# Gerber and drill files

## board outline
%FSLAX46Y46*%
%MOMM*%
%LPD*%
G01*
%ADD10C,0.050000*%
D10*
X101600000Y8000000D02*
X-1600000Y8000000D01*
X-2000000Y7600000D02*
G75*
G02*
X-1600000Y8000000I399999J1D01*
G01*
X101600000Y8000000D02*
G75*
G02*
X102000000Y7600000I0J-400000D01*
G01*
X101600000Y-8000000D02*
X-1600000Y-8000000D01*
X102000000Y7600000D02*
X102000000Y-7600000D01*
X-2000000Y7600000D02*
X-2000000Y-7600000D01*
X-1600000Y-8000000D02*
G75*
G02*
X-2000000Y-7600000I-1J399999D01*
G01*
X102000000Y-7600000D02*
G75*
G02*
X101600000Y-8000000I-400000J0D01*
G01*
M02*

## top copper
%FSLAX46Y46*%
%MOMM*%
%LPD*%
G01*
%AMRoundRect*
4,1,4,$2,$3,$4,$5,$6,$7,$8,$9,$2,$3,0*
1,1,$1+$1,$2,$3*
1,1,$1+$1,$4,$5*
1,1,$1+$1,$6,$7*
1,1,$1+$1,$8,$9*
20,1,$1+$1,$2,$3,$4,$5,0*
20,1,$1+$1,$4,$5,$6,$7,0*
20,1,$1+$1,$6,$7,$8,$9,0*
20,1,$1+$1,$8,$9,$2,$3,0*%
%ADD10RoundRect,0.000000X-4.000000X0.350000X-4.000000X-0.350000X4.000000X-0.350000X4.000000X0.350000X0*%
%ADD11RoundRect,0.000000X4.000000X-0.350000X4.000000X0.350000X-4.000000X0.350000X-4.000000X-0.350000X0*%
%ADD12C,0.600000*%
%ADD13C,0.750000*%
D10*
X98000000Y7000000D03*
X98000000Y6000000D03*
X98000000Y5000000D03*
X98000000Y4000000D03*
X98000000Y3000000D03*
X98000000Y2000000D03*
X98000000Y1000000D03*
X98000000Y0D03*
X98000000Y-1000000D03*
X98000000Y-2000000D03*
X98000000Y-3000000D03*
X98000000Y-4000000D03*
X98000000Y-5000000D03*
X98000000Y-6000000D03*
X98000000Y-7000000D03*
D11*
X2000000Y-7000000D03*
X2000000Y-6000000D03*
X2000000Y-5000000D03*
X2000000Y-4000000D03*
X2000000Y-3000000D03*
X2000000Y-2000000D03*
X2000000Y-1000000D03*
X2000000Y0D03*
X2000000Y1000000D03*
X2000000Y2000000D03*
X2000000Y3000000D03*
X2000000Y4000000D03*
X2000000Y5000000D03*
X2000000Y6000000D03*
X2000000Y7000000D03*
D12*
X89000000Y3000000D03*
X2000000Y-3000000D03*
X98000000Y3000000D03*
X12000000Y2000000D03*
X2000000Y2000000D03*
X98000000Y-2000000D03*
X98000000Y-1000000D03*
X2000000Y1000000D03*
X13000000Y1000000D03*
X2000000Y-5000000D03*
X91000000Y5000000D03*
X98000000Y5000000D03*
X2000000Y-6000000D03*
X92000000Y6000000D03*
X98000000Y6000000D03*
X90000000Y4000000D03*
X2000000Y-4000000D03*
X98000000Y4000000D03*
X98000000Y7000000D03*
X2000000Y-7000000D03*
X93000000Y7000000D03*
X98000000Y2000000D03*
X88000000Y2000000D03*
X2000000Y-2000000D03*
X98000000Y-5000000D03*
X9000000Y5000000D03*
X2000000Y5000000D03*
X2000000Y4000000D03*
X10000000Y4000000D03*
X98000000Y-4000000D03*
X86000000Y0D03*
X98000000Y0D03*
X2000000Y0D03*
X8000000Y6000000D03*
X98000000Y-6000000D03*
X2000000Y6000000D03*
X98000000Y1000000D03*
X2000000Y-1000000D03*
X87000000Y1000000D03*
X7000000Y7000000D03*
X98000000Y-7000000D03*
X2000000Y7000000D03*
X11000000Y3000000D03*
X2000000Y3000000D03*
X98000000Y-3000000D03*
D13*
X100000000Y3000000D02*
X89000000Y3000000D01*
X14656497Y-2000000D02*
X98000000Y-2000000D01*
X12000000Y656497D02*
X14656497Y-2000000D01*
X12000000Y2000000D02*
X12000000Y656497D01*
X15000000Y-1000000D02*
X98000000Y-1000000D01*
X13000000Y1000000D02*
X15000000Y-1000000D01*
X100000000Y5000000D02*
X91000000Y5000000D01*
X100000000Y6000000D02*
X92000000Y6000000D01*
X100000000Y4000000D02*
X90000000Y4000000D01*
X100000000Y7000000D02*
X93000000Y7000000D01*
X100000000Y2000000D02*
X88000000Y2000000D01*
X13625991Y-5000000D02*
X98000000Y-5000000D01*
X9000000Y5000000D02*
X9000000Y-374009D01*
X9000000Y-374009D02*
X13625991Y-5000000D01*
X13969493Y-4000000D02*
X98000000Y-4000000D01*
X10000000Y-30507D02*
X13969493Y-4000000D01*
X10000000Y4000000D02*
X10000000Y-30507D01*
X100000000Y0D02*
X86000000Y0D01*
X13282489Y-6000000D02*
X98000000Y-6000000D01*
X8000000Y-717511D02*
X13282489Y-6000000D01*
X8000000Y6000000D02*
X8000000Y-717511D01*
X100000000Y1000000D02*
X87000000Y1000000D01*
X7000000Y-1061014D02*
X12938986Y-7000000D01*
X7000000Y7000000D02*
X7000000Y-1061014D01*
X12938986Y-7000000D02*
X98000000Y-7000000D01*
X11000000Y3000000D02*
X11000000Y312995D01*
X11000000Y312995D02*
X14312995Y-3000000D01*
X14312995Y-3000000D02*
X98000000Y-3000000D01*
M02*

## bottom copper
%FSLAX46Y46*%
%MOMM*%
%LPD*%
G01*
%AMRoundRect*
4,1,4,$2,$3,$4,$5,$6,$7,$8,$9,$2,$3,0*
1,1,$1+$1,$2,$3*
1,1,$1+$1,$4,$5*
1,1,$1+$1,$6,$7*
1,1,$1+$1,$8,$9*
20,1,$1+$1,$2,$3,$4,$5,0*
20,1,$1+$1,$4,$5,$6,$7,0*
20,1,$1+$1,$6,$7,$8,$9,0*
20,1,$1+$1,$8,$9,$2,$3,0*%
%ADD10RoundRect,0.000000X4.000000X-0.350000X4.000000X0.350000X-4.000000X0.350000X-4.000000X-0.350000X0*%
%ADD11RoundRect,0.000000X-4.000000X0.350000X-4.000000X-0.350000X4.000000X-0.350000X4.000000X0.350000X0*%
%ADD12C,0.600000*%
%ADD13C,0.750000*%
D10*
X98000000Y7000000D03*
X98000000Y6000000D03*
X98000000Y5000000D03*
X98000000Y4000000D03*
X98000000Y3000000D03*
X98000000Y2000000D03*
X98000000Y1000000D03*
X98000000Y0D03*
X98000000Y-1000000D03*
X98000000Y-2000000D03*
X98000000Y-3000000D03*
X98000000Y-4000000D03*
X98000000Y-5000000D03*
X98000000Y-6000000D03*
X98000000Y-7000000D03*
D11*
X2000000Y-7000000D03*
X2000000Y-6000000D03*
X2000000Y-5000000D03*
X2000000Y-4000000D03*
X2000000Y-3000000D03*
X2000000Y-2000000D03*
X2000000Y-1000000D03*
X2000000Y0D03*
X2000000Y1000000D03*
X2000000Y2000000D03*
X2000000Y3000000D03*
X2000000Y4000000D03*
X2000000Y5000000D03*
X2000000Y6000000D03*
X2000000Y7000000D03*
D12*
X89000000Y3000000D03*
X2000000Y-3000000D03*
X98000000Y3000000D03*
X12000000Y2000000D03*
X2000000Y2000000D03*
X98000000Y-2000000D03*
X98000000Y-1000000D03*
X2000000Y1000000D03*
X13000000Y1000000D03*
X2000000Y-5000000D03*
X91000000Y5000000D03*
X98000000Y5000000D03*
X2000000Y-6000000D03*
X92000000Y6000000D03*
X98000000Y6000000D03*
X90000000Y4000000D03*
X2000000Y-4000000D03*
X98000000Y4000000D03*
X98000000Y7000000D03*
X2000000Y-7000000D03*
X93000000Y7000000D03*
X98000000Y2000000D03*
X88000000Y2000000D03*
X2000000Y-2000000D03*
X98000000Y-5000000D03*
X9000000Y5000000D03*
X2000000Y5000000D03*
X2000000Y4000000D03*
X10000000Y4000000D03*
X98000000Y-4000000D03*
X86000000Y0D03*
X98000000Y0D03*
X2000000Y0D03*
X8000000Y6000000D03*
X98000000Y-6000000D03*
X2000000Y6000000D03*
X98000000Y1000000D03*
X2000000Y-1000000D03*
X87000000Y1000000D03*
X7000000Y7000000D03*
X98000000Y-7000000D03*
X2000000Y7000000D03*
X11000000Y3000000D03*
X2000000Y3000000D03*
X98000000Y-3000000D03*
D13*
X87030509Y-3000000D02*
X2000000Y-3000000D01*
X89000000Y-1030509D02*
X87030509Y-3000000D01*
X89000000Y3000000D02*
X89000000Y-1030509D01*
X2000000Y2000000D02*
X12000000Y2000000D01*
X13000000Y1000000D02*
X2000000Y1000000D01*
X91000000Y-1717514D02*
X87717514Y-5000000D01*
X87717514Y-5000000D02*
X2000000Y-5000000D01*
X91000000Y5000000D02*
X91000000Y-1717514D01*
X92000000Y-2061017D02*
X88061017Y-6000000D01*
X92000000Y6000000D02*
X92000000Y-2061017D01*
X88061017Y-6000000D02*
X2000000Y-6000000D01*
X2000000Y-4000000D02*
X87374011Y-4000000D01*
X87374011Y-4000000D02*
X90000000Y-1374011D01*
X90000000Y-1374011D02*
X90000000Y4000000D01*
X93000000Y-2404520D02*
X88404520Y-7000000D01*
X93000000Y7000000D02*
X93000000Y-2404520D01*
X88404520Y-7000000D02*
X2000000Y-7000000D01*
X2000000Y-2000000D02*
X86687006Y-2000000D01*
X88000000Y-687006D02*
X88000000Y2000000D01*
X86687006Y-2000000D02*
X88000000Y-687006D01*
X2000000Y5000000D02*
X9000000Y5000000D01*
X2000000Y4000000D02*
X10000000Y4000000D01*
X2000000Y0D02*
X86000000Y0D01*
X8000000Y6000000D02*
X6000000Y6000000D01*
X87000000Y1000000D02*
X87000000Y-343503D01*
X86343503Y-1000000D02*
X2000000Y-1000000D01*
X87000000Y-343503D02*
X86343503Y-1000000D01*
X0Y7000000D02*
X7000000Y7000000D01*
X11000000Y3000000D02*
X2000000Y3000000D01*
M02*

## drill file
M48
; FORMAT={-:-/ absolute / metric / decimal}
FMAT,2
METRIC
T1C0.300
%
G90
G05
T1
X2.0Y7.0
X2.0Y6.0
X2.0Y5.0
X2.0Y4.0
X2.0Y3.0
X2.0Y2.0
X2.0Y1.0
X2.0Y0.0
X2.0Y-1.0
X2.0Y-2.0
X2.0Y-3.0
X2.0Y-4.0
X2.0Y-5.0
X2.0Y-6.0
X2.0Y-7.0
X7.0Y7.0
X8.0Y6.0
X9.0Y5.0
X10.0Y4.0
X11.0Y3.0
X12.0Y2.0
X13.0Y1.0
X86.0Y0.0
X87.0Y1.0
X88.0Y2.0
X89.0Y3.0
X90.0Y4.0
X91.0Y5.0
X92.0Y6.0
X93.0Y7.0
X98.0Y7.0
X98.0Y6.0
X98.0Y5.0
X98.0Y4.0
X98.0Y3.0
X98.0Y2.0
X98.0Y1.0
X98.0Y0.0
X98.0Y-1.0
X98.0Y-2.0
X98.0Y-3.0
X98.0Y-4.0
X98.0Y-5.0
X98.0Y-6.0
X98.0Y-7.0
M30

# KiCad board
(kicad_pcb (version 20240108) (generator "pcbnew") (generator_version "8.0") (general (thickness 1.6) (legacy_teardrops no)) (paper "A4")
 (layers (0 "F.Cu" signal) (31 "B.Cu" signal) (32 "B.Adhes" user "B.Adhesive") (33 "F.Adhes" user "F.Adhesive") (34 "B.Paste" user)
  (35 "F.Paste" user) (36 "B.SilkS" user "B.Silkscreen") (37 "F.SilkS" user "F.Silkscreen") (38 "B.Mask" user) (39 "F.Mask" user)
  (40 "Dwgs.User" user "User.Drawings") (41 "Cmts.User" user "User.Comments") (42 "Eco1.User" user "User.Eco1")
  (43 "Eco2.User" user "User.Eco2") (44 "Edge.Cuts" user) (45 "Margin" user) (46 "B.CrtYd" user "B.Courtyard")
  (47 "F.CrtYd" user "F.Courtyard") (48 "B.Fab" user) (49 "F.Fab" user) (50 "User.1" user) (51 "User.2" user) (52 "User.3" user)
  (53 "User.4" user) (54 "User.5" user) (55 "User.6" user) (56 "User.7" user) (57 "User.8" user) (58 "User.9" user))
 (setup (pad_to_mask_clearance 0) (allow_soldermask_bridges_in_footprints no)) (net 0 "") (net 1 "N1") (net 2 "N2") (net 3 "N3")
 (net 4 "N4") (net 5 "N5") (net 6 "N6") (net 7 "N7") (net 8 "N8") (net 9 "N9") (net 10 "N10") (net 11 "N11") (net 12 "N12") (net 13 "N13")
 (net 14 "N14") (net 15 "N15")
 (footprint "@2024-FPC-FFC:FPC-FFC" (layer "F.Cu") (at 98 0 -90)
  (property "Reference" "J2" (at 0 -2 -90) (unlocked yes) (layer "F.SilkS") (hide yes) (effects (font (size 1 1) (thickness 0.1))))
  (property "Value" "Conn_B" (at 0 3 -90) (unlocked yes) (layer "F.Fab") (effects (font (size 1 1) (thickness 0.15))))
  (pad "1" smd roundrect (at -7 0 270) (size 0.7 8) (layers "F.Cu" "F.Paste" "B.SilkS" "F.Mask") (roundrect_rratio 0) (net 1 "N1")
   (thermal_bridge_angle 45))
  (pad "1" smd roundrect (at -7 0 90) (size 0.7 8) (layers "B.Cu" "B.Paste" "F.SilkS" "B.Mask") (roundrect_rratio 0) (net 1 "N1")
   (thermal_bridge_angle 45))
  (pad "2" smd roundrect (at -6 0 270) (size 0.7 8) (layers "F.Cu" "F.Paste" "B.SilkS" "F.Mask") (roundrect_rratio 0) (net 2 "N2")
   (thermal_bridge_angle 45))
  (pad "2" smd roundrect (at -6 0 90) (size 0.7 8) (layers "B.Cu" "B.Paste" "F.SilkS" "B.Mask") (roundrect_rratio 0) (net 2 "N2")
   (thermal_bridge_angle 45))
  (pad "3" smd roundrect (at -5 0 270) (size 0.7 8) (layers "F.Cu" "F.Paste" "B.SilkS" "F.Mask") (roundrect_rratio 0) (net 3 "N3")
   (thermal_bridge_angle 45))
  (pad "3" smd roundrect (at -5 0 90) (size 0.7 8) (layers "B.Cu" "B.Paste" "F.SilkS" "B.Mask") (roundrect_rratio 0) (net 3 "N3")
   (thermal_bridge_angle 45))
  (pad "4" smd roundrect (at -4 0 270) (size 0.7 8) (layers "F.Cu" "F.Paste" "B.SilkS" "F.Mask") (roundrect_rratio 0) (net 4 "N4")
   (thermal_bridge_angle 45))
  (pad "4" smd roundrect (at -4 0 90) (size 0.7 8) (layers "B.Cu" "B.Paste" "F.SilkS" "B.Mask") (roundrect_rratio 0) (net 4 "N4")
   (thermal_bridge_angle 45))
  (pad "5" smd roundrect (at -3 0 270) (size 0.7 8) (layers "F.Cu" "F.Paste" "B.SilkS" "F.Mask") (roundrect_rratio 0) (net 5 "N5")
   (thermal_bridge_angle 45))
  (pad "5" smd roundrect (at -3 0 90) (size 0.7 8) (layers "B.Cu" "B.Paste" "F.SilkS" "B.Mask") (roundrect_rratio 0) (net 5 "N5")
   (thermal_bridge_angle 45))
  (pad "6" smd roundrect (at -2 0 270) (size 0.7 8) (layers "F.Cu" "F.Paste" "B.SilkS" "F.Mask") (roundrect_rratio 0) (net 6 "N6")
   (thermal_bridge_angle 45))
  (pad "6" smd roundrect (at -2 0 90) (size 0.7 8) (layers "B.Cu" "B.Paste" "F.SilkS" "B.Mask") (roundrect_rratio 0) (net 6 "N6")
   (thermal_bridge_angle 45))
  (pad "7" smd roundrect (at -1 0 270) (size 0.7 8) (layers "F.Cu" "F.Paste" "B.SilkS" "F.Mask") (roundrect_rratio 0) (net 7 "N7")
   (thermal_bridge_angle 45))
  (pad "7" smd roundrect (at -1 0 90) (size 0.7 8) (layers "B.Cu" "B.Paste" "F.SilkS" "B.Mask") (roundrect_rratio 0) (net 7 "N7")
   (thermal_bridge_angle 45))
  (pad "8" smd roundrect (at 0 0 270) (size 0.7 8) (layers "F.Cu" "F.Paste" "B.SilkS" "F.Mask") (roundrect_rratio 0) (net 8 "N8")
   (thermal_bridge_angle 45))
  (pad "8" smd roundrect (at 0 0 90) (size 0.7 8) (layers "B.Cu" "B.Paste" "F.SilkS" "B.Mask") (roundrect_rratio 0) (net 8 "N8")
   (thermal_bridge_angle 45))
  (pad "9" smd roundrect (at 1 0 270) (size 0.7 8) (layers "F.Cu" "F.Paste" "B.SilkS" "F.Mask") (roundrect_rratio 0) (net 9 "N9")
   (thermal_bridge_angle 45))
  (pad "9" smd roundrect (at 1 0 90) (size 0.7 8) (layers "B.Cu" "B.Paste" "F.SilkS" "B.Mask") (roundrect_rratio 0) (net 9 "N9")
   (thermal_bridge_angle 45))
  (pad "10" smd roundrect (at 2 0 270) (size 0.7 8) (layers "F.Cu" "F.Paste" "B.SilkS" "F.Mask") (roundrect_rratio 0) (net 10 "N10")
   (thermal_bridge_angle 45))
  (pad "10" smd roundrect (at 2 0 90) (size 0.7 8) (layers "B.Cu" "B.Paste" "F.SilkS" "B.Mask") (roundrect_rratio 0) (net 10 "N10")
   (thermal_bridge_angle 45))
  (pad "11" smd roundrect (at 3 0 270) (size 0.7 8) (layers "F.Cu" "F.Paste" "B.SilkS" "F.Mask") (roundrect_rratio 0) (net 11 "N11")
   (thermal_bridge_angle 45))
  (pad "11" smd roundrect (at 3 0 90) (size 0.7 8) (layers "B.Cu" "B.Paste" "F.SilkS" "B.Mask") (roundrect_rratio 0) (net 11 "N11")
   (thermal_bridge_angle 45))
  (pad "12" smd roundrect (at 4 0 270) (size 0.7 8) (layers "F.Cu" "F.Paste" "B.SilkS" "F.Mask") (roundrect_rratio 0) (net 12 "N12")
   (thermal_bridge_angle 45))
  (pad "12" smd roundrect (at 4 0 90) (size 0.7 8) (layers "B.Cu" "B.Paste" "F.SilkS" "B.Mask") (roundrect_rratio 0) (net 12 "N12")
   (thermal_bridge_angle 45))
  (pad "13" smd roundrect (at 5 0 270) (size 0.7 8) (layers "F.Cu" "F.Paste" "B.SilkS" "F.Mask") (roundrect_rratio 0) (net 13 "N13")
   (thermal_bridge_angle 45))
  (pad "13" smd roundrect (at 5 0 90) (size 0.7 8) (layers "B.Cu" "B.Paste" "F.SilkS" "B.Mask") (roundrect_rratio 0) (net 13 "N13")
   (thermal_bridge_angle 45))
  (pad "14" smd roundrect (at 6 0 270) (size 0.7 8) (layers "F.Cu" "F.Paste" "B.SilkS" "F.Mask") (roundrect_rratio 0) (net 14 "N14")
   (thermal_bridge_angle 45))
  (pad "14" smd roundrect (at 6 0 90) (size 0.7 8) (layers "B.Cu" "B.Paste" "F.SilkS" "B.Mask") (roundrect_rratio 0) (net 14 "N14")
   (thermal_bridge_angle 45))
  (pad "15" smd roundrect (at 7 0 270) (size 0.7 8) (layers "F.Cu" "F.Paste" "B.SilkS" "F.Mask") (roundrect_rratio 0) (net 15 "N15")
   (thermal_bridge_angle 45))
  (pad "15" smd roundrect (at 7 0 90) (size 0.7 8) (layers "B.Cu" "B.Paste" "F.SilkS" "B.Mask") (roundrect_rratio 0) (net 15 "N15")
   (thermal_bridge_angle 45)))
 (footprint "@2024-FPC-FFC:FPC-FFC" (layer "F.Cu") (at 2 0 90)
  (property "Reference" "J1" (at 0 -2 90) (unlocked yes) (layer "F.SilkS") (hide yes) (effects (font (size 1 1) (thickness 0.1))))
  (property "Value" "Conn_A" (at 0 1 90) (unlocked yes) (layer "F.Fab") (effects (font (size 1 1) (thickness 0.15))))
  (pad "1" smd roundrect (at -7 0 90) (size 0.7 8) (layers "F.Cu" "F.Paste" "B.SilkS" "F.Mask") (roundrect_rratio 0) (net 1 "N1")
   (thermal_bridge_angle 45))
  (pad "1" smd roundrect (at -7 0 270) (size 0.7 8) (layers "B.Cu" "B.Paste" "F.SilkS" "B.Mask") (roundrect_rratio 0) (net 1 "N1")
   (thermal_bridge_angle 45))
  (pad "2" smd roundrect (at -6 0 90) (size 0.7 8) (layers "F.Cu" "F.Paste" "B.SilkS" "F.Mask") (roundrect_rratio 0) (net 2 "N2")
   (thermal_bridge_angle 45))
  (pad "2" smd roundrect (at -6 0 270) (size 0.7 8) (layers "B.Cu" "B.Paste" "F.SilkS" "B.Mask") (roundrect_rratio 0) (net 2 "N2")
   (thermal_bridge_angle 45))
  (pad "3" smd roundrect (at -5 0 90) (size 0.7 8) (layers "F.Cu" "F.Paste" "B.SilkS" "F.Mask") (roundrect_rratio 0) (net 3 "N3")
   (thermal_bridge_angle 45))
  (pad "3" smd roundrect (at -5 0 270) (size 0.7 8) (layers "B.Cu" "B.Paste" "F.SilkS" "B.Mask") (roundrect_rratio 0) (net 3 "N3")
   (thermal_bridge_angle 45))
  (pad "4" smd roundrect (at -4 0 90) (size 0.7 8) (layers "F.Cu" "F.Paste" "B.SilkS" "F.Mask") (roundrect_rratio 0) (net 4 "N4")
   (thermal_bridge_angle 45))
  (pad "4" smd roundrect (at -4 0 270) (size 0.7 8) (layers "B.Cu" "B.Paste" "F.SilkS" "B.Mask") (roundrect_rratio 0) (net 4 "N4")
   (thermal_bridge_angle 45))
  (pad "5" smd roundrect (at -3 0 90) (size 0.7 8) (layers "F.Cu" "F.Paste" "B.SilkS" "F.Mask") (roundrect_rratio 0) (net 5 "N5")
   (thermal_bridge_angle 45))
  (pad "5" smd roundrect (at -3 0 270) (size 0.7 8) (layers "B.Cu" "B.Paste" "F.SilkS" "B.Mask") (roundrect_rratio 0) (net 5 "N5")
   (thermal_bridge_angle 45))
  (pad "6" smd roundrect (at -2 0 90) (size 0.7 8) (layers "F.Cu" "F.Paste" "B.SilkS" "F.Mask") (roundrect_rratio 0) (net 6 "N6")
   (thermal_bridge_angle 45))
  (pad "6" smd roundrect (at -2 0 270) (size 0.7 8) (layers "B.Cu" "B.Paste" "F.SilkS" "B.Mask") (roundrect_rratio 0) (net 6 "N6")
   (thermal_bridge_angle 45))
  (pad "7" smd roundrect (at -1 0 90) (size 0.7 8) (layers "F.Cu" "F.Paste" "B.SilkS" "F.Mask") (roundrect_rratio 0) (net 7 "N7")
   (thermal_bridge_angle 45))
  (pad "7" smd roundrect (at -1 0 270) (size 0.7 8) (layers "B.Cu" "B.Paste" "F.SilkS" "B.Mask") (roundrect_rratio 0) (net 7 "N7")
   (thermal_bridge_angle 45))
  (pad "8" smd roundrect (at 0 0 90) (size 0.7 8) (layers "F.Cu" "F.Paste" "B.SilkS" "F.Mask") (roundrect_rratio 0) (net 8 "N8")
   (thermal_bridge_angle 45))
  (pad "8" smd roundrect (at 0 0 270) (size 0.7 8) (layers "B.Cu" "B.Paste" "F.SilkS" "B.Mask") (roundrect_rratio 0) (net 8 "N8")
   (thermal_bridge_angle 45))
  (pad "9" smd roundrect (at 1 0 90) (size 0.7 8) (layers "F.Cu" "F.Paste" "B.SilkS" "F.Mask") (roundrect_rratio 0) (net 9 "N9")
   (thermal_bridge_angle 45))
  (pad "9" smd roundrect (at 1 0 270) (size 0.7 8) (layers "B.Cu" "B.Paste" "F.SilkS" "B.Mask") (roundrect_rratio 0) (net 9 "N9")
   (thermal_bridge_angle 45))
  (pad "10" smd roundrect (at 2 0 90) (size 0.7 8) (layers "F.Cu" "F.Paste" "B.SilkS" "F.Mask") (roundrect_rratio 0) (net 10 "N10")
   (thermal_bridge_angle 45))
  (pad "10" smd roundrect (at 2 0 270) (size 0.7 8) (layers "B.Cu" "B.Paste" "F.SilkS" "B.Mask") (roundrect_rratio 0) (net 10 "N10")
   (thermal_bridge_angle 45))
  (pad "11" smd roundrect (at 3 0 90) (size 0.7 8) (layers "F.Cu" "F.Paste" "B.SilkS" "F.Mask") (roundrect_rratio 0) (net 11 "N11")
   (thermal_bridge_angle 45))
  (pad "11" smd roundrect (at 3 0 270) (size 0.7 8) (layers "B.Cu" "B.Paste" "F.SilkS" "B.Mask") (roundrect_rratio 0) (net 11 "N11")
   (thermal_bridge_angle 45))
  (pad "12" smd roundrect (at 4 0 90) (size 0.7 8) (layers "F.Cu" "F.Paste" "B.SilkS" "F.Mask") (roundrect_rratio 0) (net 12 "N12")
   (thermal_bridge_angle 45))
  (pad "12" smd roundrect (at 4 0 270) (size 0.7 8) (layers "B.Cu" "B.Paste" "F.SilkS" "B.Mask") (roundrect_rratio 0) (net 12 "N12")
   (thermal_bridge_angle 45))
  (pad "13" smd roundrect (at 5 0 90) (size 0.7 8) (layers "F.Cu" "F.Paste" "B.SilkS" "F.Mask") (roundrect_rratio 0) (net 13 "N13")
   (thermal_bridge_angle 45))
  (pad "13" smd roundrect (at 5 0 270) (size 0.7 8) (layers "B.Cu" "B.Paste" "F.SilkS" "B.Mask") (roundrect_rratio 0) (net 13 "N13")
   (thermal_bridge_angle 45))
  (pad "14" smd roundrect (at 6 0 90) (size 0.7 8) (layers "F.Cu" "F.Paste" "B.SilkS" "F.Mask") (roundrect_rratio 0) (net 14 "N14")
   (thermal_bridge_angle 45))
  (pad "14" smd roundrect (at 6 0 270) (size 0.7 8) (layers "B.Cu" "B.Paste" "F.SilkS" "B.Mask") (roundrect_rratio 0) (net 14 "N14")
   (thermal_bridge_angle 45))
  (pad "15" smd roundrect (at 7 0 90) (size 0.7 8) (layers "F.Cu" "F.Paste" "B.SilkS" "F.Mask") (roundrect_rratio 0) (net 15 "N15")
   (thermal_bridge_angle 45))
  (pad "15" smd roundrect (at 7 0 270) (size 0.7 8) (layers "B.Cu" "B.Paste" "F.SilkS" "B.Mask") (roundrect_rratio 0) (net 15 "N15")
   (thermal_bridge_angle 45)))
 (gr_line (start 101.6 -8) (end -1.6 -8) (stroke (width 0.05) (type default)) (layer "Edge.Cuts"))
 (gr_arc (start -2 -7.6) (mid -1.882843 -7.882843) (end -1.6 -8) (stroke (width 0.05) (type default)) (layer "Edge.Cuts"))
 (gr_arc (start 101.6 -8) (mid 101.882843 -7.882843) (end 102 -7.6) (stroke (width 0.05) (type default)) (layer "Edge.Cuts"))
 (gr_line (start 101.6 8) (end -1.6 8) (stroke (width 0.05) (type default)) (layer "Edge.Cuts"))
 (gr_line (start 102 -7.6) (end 102 7.6) (stroke (width 0.05) (type default)) (layer "Edge.Cuts"))
 (gr_line (start -2 -7.6) (end -2 7.6) (stroke (width 0.05) (type default)) (layer "Edge.Cuts"))
 (gr_arc (start -1.6 8) (mid -1.882843 7.882843) (end -2 7.6) (stroke (width 0.05) (type default)) (layer "Edge.Cuts"))
 (gr_arc (start 102 7.6) (mid 101.882843 7.882843) (end 101.6 8) (stroke (width 0.05) (type default)) (layer "Edge.Cuts"))
 (segment (start 100 -3) (end 89 -3) (width 0.75) (layer "F.Cu") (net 5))
 (via (at 89 -3) (size 0.6) (drill 0.3) (layers "F.Cu" "B.Cu") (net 5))
 (via (at 2 3) (size 0.6) (drill 0.3) (layers "F.Cu" "B.Cu") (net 5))
 (via (at 98 -3) (size 0.6) (drill 0.3) (layers "F.Cu" "B.Cu") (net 5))
 (segment (start 87.030509 3) (end 2 3) (width 0.75) (layer "B.Cu") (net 5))
 (segment (start 89 1.030509) (end 87.030509 3) (width 0.75) (layer "B.Cu") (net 5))
 (segment (start 89 -3) (end 89 1.030509) (width 0.75) (layer "B.Cu") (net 5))
 (segment (start 14.656497 2) (end 98 2) (width 0.75) (layer "F.Cu") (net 10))
 (segment (start 12 -0.656497) (end 14.656497 2) (width 0.75) (layer "F.Cu") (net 10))
 (segment (start 12 -2) (end 12 -0.656497) (width 0.75) (layer "F.Cu") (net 10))
 (via (at 12 -2) (size 0.6) (drill 0.3) (layers "F.Cu" "B.Cu") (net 10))
 (via (at 2 -2) (size 0.6) (drill 0.3) (layers "F.Cu" "B.Cu") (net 10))
 (via (at 98 2) (size 0.6) (drill 0.3) (layers "F.Cu" "B.Cu") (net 10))
 (segment (start 2 -2) (end 12 -2) (width 0.75) (layer "B.Cu") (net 10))
 (segment (start 15 1) (end 98 1) (width 0.75) (layer "F.Cu") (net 9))
 (segment (start 13 -1) (end 15 1) (width 0.75) (layer "F.Cu") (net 9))
 (via (at 98 1) (size 0.6) (drill 0.3) (layers "F.Cu" "B.Cu") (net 9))
 (via (at 2 -1) (size 0.6) (drill 0.3) (layers "F.Cu" "B.Cu") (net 9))
 (via (at 13 -1) (size 0.6) (drill 0.3) (layers "F.Cu" "B.Cu") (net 9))
 (segment (start 13 -1) (end 2 -1) (width 0.75) (layer "B.Cu") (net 9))
 (segment (start 100 -5) (end 91 -5) (width 0.75) (layer "F.Cu") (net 3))
 (via (at 2 5) (size 0.6) (drill 0.3) (layers "F.Cu" "B.Cu") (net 3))
 (via (at 91 -5) (size 0.6) (drill 0.3) (layers "F.Cu" "B.Cu") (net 3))
 (via (at 98 -5) (size 0.6) (drill 0.3) (layers "F.Cu" "B.Cu") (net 3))
 (segment (start 91 1.717514) (end 87.717514 5) (width 0.75) (layer "B.Cu") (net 3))
 (segment (start 87.717514 5) (end 2 5) (width 0.75) (layer "B.Cu") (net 3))
 (segment (start 91 -5) (end 91 1.717514) (width 0.75) (layer "B.Cu") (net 3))
 (segment (start 100 -6) (end 92 -6) (width 0.75) (layer "F.Cu") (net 2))
 (via (at 2 6) (size 0.6) (drill 0.3) (layers "F.Cu" "B.Cu") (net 2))
 (via (at 92 -6) (size 0.6) (drill 0.3) (layers "F.Cu" "B.Cu") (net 2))
 (via (at 98 -6) (size 0.6) (drill 0.3) (layers "F.Cu" "B.Cu") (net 2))
 (segment (start 92 2.061017) (end 88.061017 6) (width 0.75) (layer "B.Cu") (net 2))
 (segment (start 92 -6) (end 92 2.061017) (width 0.75) (layer "B.Cu") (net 2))
 (segment (start 88.061017 6) (end 2 6) (width 0.75) (layer "B.Cu") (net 2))
 (segment (start 100 -4) (end 90 -4) (width 0.75) (layer "F.Cu") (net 4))
 (via (at 90 -4) (size 0.6) (drill 0.3) (layers "F.Cu" "B.Cu") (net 4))
 (via (at 2 4) (size 0.6) (drill 0.3) (layers "F.Cu" "B.Cu") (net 4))
 (via (at 98 -4) (size 0.6) (drill 0.3) (layers "F.Cu" "B.Cu") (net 4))
 (segment (start 2 4) (end 87.374011 4) (width 0.75) (layer "B.Cu") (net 4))
 (segment (start 87.374011 4) (end 90 1.374011) (width 0.75) (layer "B.Cu") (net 4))
 (segment (start 90 1.374011) (end 90 -4) (width 0.75) (layer "B.Cu") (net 4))
 (segment (start 100 -7) (end 93 -7) (width 0.75) (layer "F.Cu") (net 1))
 (via (at 98 -7) (size 0.6) (drill 0.3) (layers "F.Cu" "B.Cu") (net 1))
 (via (at 2 7) (size 0.6) (drill 0.3) (layers "F.Cu" "B.Cu") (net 1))
 (via (at 93 -7) (size 0.6) (drill 0.3) (layers "F.Cu" "B.Cu") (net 1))
 (segment (start 93 2.40452) (end 88.40452 7) (width 0.75) (layer "B.Cu") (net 1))
 (segment (start 93 -7) (end 93 2.40452) (width 0.75) (layer "B.Cu") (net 1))
 (segment (start 88.40452 7) (end 2 7) (width 0.75) (layer "B.Cu") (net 1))
 (segment (start 100 -2) (end 88 -2) (width 0.75) (layer "F.Cu") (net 6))
 (via (at 98 -2) (size 0.6) (drill 0.3) (layers "F.Cu" "B.Cu") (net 6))
 (via (at 88 -2) (size 0.6) (drill 0.3) (layers "F.Cu" "B.Cu") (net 6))
 (via (at 2 2) (size 0.6) (drill 0.3) (layers "F.Cu" "B.Cu") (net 6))
 (segment (start 2 2) (end 86.687006 2) (width 0.75) (layer "B.Cu") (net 6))
 (segment (start 88 0.687006) (end 88 -2) (width 0.75) (layer "B.Cu") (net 6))
 (segment (start 86.687006 2) (end 88 0.687006) (width 0.75) (layer "B.Cu") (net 6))
 (segment (start 13.625991 5) (end 98 5) (width 0.75) (layer "F.Cu") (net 13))
 (segment (start 9 -5) (end 9 0.374009) (width 0.75) (layer "F.Cu") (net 13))
 (segment (start 9 0.374009) (end 13.625991 5) (width 0.75) (layer "F.Cu") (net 13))
 (via (at 98 5) (size 0.6) (drill 0.3) (layers "F.Cu" "B.Cu") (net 13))
 (via (at 9 -5) (size 0.6) (drill 0.3) (layers "F.Cu" "B.Cu") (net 13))
 (via (at 2 -5) (size 0.6) (drill 0.3) (layers "F.Cu" "B.Cu") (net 13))
 (segment (start 2 -5) (end 9 -5) (width 0.75) (layer "B.Cu") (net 13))
 (segment (start 13.969493 4) (end 98 4) (width 0.75) (layer "F.Cu") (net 12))
 (segment (start 10 0.030507) (end 13.969493 4) (width 0.75) (layer "F.Cu") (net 12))
 (segment (start 10 -4) (end 10 0.030507) (width 0.75) (layer "F.Cu") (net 12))
 (via (at 2 -4) (size 0.6) (drill 0.3) (layers "F.Cu" "B.Cu") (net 12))
 (via (at 10 -4) (size 0.6) (drill 0.3) (layers "F.Cu" "B.Cu") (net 12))
 (via (at 98 4) (size 0.6) (drill 0.3) (layers "F.Cu" "B.Cu") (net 12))
 (segment (start 2 -4) (end 10 -4) (width 0.75) (layer "B.Cu") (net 12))
 (segment (start 100 0) (end 86 0) (width 0.75) (layer "F.Cu") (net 8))
 (via (at 86 0) (size 0.6) (drill 0.3) (layers "F.Cu" "B.Cu") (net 8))
 (via (at 98 0) (size 0.6) (drill 0.3) (layers "F.Cu" "B.Cu") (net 8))
 (via (at 2 0) (size 0.6) (drill 0.3) (layers "F.Cu" "B.Cu") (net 8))
 (segment (start 2 0) (end 86 0) (width 0.75) (layer "B.Cu") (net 8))
 (segment (start 13.282489 6) (end 98 6) (width 0.75) (layer "F.Cu") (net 14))
 (segment (start 8 0.717511) (end 13.282489 6) (width 0.75) (layer "F.Cu") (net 14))
 (segment (start 8 -6) (end 8 0.717511) (width 0.75) (layer "F.Cu") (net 14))
 (via (at 8 -6) (size 0.6) (drill 0.3) (layers "F.Cu" "B.Cu") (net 14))
 (via (at 98 6) (size 0.6) (drill 0.3) (layers "F.Cu" "B.Cu") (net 14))
 (via (at 2 -6) (size 0.6) (drill 0.3) (layers "F.Cu" "B.Cu") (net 14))
 (segment (start 8 -6) (end 6 -6) (width 0.75) (layer "B.Cu") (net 14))
 (segment (start 100 -1) (end 87 -1) (width 0.75) (layer "F.Cu") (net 7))
 (via (at 98 -1) (size 0.6) (drill 0.3) (layers "F.Cu" "B.Cu") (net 7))
 (via (at 2 1) (size 0.6) (drill 0.3) (layers "F.Cu" "B.Cu") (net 7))
 (via (at 87 -1) (size 0.6) (drill 0.3) (layers "F.Cu" "B.Cu") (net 7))
 (segment (start 87 -1) (end 87 0.343503) (width 0.75) (layer "B.Cu") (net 7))
 (segment (start 86.343503 1) (end 2 1) (width 0.75) (layer "B.Cu") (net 7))
 (segment (start 87 0.343503) (end 86.343503 1) (width 0.75) (layer "B.Cu") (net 7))
 (segment (start 7 1.061014) (end 12.938986 7) (width 0.75) (layer "F.Cu") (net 15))
 (segment (start 7 -7) (end 7 1.061014) (width 0.75) (layer "F.Cu") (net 15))
 (segment (start 12.938986 7) (end 98 7) (width 0.75) (layer "F.Cu") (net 15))
 (via (at 7 -7) (size 0.6) (drill 0.3) (layers "F.Cu" "B.Cu") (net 15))
 (via (at 98 7) (size 0.6) (drill 0.3) (layers "F.Cu" "B.Cu") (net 15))
 (via (at 2 -7) (size 0.6) (drill 0.3) (layers "F.Cu" "B.Cu") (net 15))
 (segment (start 0 -7) (end 7 -7) (width 0.75) (layer "B.Cu") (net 15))
 (segment (start 11 -3) (end 11 -0.312995) (width 0.75) (layer "F.Cu") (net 11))
 (segment (start 11 -0.312995) (end 14.312995 3) (width 0.75) (layer "F.Cu") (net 11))
 (segment (start 14.312995 3) (end 98 3) (width 0.75) (layer "F.Cu") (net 11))
 (via (at 11 -3) (size 0.6) (drill 0.3) (layers "F.Cu" "B.Cu") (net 11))
 (via (at 2 -3) (size 0.6) (drill 0.3) (layers "F.Cu" "B.Cu") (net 11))
 (via (at 98 3) (size 0.6) (drill 0.3) (layers "F.Cu" "B.Cu") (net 11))
 (segment (start 11 -3) (end 2 -3) (width 0.75) (layer "B.Cu") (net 11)))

